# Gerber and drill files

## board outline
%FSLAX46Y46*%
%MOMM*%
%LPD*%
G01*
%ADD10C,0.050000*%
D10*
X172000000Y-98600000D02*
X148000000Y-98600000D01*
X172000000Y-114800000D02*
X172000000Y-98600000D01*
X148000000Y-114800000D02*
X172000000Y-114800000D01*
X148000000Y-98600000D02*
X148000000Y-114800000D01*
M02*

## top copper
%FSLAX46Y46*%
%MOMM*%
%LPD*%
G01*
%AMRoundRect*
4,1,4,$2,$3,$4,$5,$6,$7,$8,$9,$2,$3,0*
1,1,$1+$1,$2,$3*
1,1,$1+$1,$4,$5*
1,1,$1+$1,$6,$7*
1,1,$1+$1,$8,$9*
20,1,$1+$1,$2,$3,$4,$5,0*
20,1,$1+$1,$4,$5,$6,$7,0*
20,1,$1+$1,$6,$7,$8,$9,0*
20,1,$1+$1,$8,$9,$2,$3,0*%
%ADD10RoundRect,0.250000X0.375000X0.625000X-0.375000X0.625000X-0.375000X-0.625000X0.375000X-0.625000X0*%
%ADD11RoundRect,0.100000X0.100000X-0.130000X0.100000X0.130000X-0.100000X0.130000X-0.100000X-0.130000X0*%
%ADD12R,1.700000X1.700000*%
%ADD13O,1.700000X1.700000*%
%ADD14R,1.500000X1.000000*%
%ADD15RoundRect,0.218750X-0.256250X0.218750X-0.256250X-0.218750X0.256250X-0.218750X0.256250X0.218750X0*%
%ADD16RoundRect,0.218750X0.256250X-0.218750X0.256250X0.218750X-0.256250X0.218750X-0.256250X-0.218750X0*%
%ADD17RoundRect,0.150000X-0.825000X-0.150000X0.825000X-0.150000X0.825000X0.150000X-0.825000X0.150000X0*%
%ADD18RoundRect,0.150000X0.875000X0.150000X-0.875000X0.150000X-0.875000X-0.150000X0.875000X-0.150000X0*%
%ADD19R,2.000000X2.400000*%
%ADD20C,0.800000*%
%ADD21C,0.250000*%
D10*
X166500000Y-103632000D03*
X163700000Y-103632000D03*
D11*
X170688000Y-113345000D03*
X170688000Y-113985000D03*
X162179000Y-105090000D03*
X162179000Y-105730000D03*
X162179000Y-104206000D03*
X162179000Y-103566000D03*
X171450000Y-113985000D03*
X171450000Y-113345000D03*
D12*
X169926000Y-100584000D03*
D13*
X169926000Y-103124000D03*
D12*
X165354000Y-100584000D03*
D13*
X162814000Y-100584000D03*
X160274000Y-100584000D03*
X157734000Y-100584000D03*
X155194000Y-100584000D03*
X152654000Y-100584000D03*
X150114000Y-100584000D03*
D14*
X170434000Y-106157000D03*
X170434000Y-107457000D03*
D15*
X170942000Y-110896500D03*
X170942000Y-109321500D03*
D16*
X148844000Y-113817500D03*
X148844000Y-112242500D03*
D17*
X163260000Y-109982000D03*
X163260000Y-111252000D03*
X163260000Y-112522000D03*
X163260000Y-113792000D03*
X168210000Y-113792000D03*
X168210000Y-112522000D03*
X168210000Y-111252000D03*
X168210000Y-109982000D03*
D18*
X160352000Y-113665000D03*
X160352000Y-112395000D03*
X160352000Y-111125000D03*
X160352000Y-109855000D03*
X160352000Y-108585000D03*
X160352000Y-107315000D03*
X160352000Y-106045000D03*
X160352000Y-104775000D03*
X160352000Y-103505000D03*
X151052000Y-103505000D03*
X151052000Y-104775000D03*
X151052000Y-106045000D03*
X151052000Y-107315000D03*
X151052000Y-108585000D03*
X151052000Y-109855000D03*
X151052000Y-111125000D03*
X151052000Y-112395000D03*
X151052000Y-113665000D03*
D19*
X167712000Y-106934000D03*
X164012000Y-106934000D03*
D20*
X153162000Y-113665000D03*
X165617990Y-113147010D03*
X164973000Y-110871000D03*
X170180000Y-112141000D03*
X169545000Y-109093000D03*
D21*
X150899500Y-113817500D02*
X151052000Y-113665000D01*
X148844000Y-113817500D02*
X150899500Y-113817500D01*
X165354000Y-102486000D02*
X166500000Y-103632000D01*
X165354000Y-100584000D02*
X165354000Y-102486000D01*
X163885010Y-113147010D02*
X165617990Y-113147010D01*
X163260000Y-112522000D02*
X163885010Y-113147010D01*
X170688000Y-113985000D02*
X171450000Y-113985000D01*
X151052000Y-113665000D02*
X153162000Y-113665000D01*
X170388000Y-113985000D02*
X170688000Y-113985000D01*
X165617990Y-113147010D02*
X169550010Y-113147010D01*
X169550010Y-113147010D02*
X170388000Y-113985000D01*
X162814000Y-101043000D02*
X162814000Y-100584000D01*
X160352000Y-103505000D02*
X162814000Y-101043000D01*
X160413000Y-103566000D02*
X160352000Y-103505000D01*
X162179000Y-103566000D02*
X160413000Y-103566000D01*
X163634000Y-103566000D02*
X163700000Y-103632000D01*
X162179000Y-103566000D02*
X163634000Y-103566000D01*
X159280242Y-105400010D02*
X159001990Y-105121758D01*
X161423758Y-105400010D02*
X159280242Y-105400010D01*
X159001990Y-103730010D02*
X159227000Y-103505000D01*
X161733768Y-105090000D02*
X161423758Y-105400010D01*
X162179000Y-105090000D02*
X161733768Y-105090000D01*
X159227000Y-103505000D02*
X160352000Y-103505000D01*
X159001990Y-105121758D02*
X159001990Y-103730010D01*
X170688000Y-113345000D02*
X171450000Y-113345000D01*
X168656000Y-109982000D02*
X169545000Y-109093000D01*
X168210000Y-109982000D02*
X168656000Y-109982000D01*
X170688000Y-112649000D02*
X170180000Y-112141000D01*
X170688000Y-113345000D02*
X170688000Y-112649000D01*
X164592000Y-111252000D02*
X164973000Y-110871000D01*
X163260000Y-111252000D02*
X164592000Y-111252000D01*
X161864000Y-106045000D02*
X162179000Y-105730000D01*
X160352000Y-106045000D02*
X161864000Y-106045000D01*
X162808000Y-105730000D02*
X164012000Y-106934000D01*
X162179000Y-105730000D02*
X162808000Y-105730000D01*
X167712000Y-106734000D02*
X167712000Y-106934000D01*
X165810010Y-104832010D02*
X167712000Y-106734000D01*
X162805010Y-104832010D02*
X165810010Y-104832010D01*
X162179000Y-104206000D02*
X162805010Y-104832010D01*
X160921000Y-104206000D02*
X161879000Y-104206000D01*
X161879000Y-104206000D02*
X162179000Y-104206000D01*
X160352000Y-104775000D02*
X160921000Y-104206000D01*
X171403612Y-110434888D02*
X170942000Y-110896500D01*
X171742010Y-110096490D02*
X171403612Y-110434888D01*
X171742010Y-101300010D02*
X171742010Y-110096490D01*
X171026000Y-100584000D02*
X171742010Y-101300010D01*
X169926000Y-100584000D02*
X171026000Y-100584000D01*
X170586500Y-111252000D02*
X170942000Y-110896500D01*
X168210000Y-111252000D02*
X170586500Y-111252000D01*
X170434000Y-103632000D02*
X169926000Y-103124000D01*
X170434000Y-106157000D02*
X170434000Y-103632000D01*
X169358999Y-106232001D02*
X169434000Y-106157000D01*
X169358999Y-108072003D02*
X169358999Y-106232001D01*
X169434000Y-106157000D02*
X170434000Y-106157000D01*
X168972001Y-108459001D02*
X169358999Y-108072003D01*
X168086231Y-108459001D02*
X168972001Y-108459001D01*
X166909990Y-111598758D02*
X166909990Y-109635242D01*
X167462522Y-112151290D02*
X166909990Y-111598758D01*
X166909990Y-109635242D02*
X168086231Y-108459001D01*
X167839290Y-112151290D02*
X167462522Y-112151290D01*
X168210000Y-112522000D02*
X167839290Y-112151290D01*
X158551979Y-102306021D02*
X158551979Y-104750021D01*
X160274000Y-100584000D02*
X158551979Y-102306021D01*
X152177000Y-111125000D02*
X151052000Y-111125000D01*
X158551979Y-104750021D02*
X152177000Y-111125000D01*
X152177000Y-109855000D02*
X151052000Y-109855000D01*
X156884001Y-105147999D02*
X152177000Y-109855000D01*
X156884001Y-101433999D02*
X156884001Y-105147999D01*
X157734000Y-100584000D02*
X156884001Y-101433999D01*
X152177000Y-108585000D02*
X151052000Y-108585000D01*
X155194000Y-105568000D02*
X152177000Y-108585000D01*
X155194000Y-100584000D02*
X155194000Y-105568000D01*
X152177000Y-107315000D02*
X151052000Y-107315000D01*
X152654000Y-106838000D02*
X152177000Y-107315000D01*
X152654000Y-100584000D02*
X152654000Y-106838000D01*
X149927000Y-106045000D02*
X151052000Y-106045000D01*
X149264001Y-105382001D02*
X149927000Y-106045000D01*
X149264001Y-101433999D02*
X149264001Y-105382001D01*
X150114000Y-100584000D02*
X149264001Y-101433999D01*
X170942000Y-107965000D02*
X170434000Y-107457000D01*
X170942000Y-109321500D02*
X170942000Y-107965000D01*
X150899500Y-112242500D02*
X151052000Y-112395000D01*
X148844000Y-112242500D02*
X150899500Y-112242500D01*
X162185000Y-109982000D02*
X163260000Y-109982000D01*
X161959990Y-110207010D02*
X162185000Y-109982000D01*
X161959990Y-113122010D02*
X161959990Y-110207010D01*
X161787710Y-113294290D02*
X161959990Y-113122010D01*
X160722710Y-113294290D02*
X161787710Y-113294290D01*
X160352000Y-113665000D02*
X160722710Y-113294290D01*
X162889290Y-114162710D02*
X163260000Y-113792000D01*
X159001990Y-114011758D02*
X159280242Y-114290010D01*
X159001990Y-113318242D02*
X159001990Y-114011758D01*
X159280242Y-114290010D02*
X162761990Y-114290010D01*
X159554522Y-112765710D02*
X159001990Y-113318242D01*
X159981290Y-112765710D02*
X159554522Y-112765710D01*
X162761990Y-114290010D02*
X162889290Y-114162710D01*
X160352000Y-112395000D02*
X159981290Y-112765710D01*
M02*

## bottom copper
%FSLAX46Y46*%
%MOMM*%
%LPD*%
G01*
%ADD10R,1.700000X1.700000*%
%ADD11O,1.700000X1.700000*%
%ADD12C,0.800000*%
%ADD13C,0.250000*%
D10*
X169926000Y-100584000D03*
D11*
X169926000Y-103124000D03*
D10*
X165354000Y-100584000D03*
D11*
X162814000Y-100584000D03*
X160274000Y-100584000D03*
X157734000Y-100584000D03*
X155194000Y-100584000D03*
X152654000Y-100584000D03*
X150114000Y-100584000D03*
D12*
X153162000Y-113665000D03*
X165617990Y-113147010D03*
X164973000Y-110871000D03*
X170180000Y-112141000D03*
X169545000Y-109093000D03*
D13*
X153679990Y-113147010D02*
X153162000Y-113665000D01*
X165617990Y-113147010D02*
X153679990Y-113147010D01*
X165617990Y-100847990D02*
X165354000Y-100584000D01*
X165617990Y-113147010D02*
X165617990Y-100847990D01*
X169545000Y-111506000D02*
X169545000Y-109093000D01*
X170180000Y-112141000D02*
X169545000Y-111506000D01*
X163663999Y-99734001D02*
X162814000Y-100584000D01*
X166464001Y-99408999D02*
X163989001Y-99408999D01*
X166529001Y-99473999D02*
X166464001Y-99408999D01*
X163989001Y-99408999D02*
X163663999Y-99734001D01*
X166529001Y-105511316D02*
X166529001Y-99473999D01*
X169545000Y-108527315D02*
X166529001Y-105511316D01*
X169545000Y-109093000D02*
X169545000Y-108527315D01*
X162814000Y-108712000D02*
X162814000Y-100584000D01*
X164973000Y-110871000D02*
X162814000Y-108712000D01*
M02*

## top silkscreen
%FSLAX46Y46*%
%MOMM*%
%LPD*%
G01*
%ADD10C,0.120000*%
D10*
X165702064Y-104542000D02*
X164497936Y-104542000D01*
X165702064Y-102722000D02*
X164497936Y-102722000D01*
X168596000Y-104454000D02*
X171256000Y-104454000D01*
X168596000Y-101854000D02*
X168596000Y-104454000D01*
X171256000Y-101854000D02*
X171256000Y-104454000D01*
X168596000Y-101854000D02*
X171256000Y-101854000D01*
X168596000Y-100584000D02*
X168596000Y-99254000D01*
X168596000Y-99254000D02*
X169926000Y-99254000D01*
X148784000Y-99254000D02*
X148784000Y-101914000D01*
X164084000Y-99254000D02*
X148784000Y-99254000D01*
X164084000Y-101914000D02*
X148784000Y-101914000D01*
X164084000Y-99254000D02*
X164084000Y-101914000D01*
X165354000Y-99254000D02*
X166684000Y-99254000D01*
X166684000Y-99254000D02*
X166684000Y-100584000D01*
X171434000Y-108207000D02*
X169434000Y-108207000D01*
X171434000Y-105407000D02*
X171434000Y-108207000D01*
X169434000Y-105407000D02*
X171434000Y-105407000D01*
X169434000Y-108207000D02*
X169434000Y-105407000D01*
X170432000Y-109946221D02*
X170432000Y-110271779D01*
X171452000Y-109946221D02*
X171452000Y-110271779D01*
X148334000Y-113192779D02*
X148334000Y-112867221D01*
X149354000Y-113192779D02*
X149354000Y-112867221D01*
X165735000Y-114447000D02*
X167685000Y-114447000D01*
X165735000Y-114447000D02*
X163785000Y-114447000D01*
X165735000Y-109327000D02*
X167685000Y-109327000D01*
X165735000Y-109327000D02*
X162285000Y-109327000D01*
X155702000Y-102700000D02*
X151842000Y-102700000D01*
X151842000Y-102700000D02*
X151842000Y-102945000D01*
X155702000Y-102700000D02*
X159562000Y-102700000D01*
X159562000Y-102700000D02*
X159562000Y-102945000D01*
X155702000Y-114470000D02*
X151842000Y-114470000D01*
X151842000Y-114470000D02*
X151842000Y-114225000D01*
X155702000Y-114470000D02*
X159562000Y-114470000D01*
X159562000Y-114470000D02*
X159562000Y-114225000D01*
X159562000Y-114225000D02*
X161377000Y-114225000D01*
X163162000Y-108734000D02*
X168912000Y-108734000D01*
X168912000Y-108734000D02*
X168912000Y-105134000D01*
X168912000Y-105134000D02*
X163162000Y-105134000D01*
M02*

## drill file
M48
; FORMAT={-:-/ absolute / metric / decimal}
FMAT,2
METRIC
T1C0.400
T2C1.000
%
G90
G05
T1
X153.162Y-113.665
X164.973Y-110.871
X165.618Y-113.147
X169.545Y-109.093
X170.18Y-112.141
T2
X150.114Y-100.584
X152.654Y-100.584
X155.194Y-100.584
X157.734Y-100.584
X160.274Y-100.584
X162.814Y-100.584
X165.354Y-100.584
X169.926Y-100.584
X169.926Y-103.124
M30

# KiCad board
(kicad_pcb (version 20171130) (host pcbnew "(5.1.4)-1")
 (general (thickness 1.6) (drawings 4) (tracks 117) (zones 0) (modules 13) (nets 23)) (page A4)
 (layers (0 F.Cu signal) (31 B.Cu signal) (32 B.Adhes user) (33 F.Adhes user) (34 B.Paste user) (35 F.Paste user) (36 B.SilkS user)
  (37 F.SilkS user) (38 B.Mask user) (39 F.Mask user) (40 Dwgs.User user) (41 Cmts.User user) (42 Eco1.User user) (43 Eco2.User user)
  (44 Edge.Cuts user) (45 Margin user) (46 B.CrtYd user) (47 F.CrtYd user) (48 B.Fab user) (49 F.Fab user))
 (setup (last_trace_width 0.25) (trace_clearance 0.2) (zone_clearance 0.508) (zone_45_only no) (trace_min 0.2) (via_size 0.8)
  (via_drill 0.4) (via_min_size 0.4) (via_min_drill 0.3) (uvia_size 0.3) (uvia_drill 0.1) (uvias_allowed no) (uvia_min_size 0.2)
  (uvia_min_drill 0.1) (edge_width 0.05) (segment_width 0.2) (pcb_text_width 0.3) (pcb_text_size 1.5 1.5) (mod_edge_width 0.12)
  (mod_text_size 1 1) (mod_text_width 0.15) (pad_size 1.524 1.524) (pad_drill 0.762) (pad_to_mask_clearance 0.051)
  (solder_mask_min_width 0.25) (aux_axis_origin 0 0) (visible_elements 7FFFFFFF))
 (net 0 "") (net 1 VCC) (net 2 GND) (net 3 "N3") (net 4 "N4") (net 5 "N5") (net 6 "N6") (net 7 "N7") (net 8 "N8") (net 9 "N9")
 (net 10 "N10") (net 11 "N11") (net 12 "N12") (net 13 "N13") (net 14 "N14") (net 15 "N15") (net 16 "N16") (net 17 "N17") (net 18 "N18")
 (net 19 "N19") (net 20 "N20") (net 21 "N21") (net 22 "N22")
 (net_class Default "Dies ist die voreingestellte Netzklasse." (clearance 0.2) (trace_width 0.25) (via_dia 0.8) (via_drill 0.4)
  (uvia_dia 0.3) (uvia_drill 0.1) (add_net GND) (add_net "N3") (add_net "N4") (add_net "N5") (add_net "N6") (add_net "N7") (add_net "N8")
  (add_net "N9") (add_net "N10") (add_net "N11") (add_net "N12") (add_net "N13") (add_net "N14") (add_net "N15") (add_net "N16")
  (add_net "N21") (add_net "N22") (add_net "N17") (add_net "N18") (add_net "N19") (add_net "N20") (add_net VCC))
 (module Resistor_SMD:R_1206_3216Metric (layer F.Cu) (at 165.1 103.632 180)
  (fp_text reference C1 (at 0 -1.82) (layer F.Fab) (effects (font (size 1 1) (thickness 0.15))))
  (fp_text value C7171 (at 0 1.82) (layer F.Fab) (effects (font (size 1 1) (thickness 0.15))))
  (fp_line (start -0.602064 -0.91) (end 0.602064 -0.91) (layer F.SilkS) (width 0.12))
  (fp_line (start -0.602064 0.91) (end 0.602064 0.91) (layer F.SilkS) (width 0.12))
  (pad 1 smd roundrect (at -1.4 0 180) (size 1.25 1.75) (layers F.Cu F.Paste F.Mask) (roundrect_rratio 0.2) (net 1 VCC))
  (pad 2 smd roundrect (at 1.4 0 180) (size 1.25 1.75) (layers F.Cu F.Paste F.Mask) (roundrect_rratio 0.2) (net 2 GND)))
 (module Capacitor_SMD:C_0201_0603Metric (layer F.Cu) (at 170.688 113.665 90)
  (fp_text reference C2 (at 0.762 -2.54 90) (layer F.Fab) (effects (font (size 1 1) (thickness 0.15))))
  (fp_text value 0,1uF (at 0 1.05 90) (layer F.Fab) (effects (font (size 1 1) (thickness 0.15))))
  (pad 2 smd roundrect (at 0.32 0 90) (size 0.46 0.4) (layers F.Cu F.Mask) (roundrect_rratio 0.25) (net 2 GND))
  (pad 1 smd roundrect (at -0.32 0 90) (size 0.46 0.4) (layers F.Cu F.Mask) (roundrect_rratio 0.25) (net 1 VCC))
  (pad "" smd roundrect (at 0.345 0 90) (size 0.318 0.36) (layers F.Paste) (roundrect_rratio 0.25))
  (pad "" smd roundrect (at -0.345 0 90) (size 0.318 0.36) (layers F.Paste) (roundrect_rratio 0.25)))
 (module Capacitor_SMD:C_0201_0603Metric (layer F.Cu) (at 162.179 105.41 90)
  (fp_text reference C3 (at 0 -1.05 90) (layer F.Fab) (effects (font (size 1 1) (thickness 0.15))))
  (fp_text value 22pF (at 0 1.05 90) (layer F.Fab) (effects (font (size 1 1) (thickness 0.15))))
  (pad 2 smd roundrect (at 0.32 0 90) (size 0.46 0.4) (layers F.Cu F.Mask) (roundrect_rratio 0.25) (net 2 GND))
  (pad 1 smd roundrect (at -0.32 0 90) (size 0.46 0.4) (layers F.Cu F.Mask) (roundrect_rratio 0.25) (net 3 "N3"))
  (pad "" smd roundrect (at 0.345 0 90) (size 0.318 0.36) (layers F.Paste) (roundrect_rratio 0.25))
  (pad "" smd roundrect (at -0.345 0 90) (size 0.318 0.36) (layers F.Paste) (roundrect_rratio 0.25)))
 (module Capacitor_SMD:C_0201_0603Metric (layer F.Cu) (at 162.179 103.886 90)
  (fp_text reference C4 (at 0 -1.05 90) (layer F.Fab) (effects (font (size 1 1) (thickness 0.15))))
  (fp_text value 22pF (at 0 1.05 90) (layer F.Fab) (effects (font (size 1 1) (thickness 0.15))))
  (pad "" smd roundrect (at -0.345 0 90) (size 0.318 0.36) (layers F.Paste) (roundrect_rratio 0.25))
  (pad "" smd roundrect (at 0.345 0 90) (size 0.318 0.36) (layers F.Paste) (roundrect_rratio 0.25))
  (pad 1 smd roundrect (at -0.32 0 90) (size 0.46 0.4) (layers F.Cu F.Mask) (roundrect_rratio 0.25) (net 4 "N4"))
  (pad 2 smd roundrect (at 0.32 0 90) (size 0.46 0.4) (layers F.Cu F.Mask) (roundrect_rratio 0.25) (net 2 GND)))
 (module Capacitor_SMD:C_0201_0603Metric (layer F.Cu) (at 171.45 113.665 90)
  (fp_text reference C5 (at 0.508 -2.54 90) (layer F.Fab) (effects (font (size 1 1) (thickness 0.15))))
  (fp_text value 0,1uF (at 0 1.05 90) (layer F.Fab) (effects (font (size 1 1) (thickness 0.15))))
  (pad "" smd roundrect (at -0.345 0 90) (size 0.318 0.36) (layers F.Paste) (roundrect_rratio 0.25))
  (pad "" smd roundrect (at 0.345 0 90) (size 0.318 0.36) (layers F.Paste) (roundrect_rratio 0.25))
  (pad 1 smd roundrect (at -0.32 0 90) (size 0.46 0.4) (layers F.Cu F.Mask) (roundrect_rratio 0.25) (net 1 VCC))
  (pad 2 smd roundrect (at 0.32 0 90) (size 0.46 0.4) (layers F.Cu F.Mask) (roundrect_rratio 0.25) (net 2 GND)))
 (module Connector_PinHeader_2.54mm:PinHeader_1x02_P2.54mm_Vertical (layer F.Cu) (at 169.926 100.584)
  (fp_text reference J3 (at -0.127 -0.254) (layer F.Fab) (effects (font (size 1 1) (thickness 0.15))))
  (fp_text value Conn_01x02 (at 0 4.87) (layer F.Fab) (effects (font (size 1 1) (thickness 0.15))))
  (fp_line (start -1.33 3.87) (end 1.33 3.87) (layer F.SilkS) (width 0.12))
  (fp_line (start -1.33 1.27) (end -1.33 3.87) (layer F.SilkS) (width 0.12))
  (fp_line (start 1.33 1.27) (end 1.33 3.87) (layer F.SilkS) (width 0.12))
  (fp_line (start -1.33 1.27) (end 1.33 1.27) (layer F.SilkS) (width 0.12))
  (fp_line (start -1.33 0) (end -1.33 -1.33) (layer F.SilkS) (width 0.12))
  (fp_line (start -1.33 -1.33) (end 0 -1.33) (layer F.SilkS) (width 0.12))
  (pad 1 thru_hole rect (at 0 0) (size 1.7 1.7) (drill 1) (layers *.Cu *.Mask) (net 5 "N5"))
  (pad 2 thru_hole oval (at 0 2.54) (size 1.7 1.7) (drill 1) (layers *.Cu *.Mask) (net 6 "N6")))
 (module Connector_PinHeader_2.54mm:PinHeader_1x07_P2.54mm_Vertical (layer F.Cu) (at 165.354 100.584 270)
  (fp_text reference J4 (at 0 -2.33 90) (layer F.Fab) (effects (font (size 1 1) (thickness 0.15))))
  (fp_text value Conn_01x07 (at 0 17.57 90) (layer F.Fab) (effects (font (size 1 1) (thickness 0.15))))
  (fp_line (start -1.33 16.57) (end 1.33 16.57) (layer F.SilkS) (width 0.12))
  (fp_line (start -1.33 1.27) (end -1.33 16.57) (layer F.SilkS) (width 0.12))
  (fp_line (start 1.33 1.27) (end 1.33 16.57) (layer F.SilkS) (width 0.12))
  (fp_line (start -1.33 1.27) (end 1.33 1.27) (layer F.SilkS) (width 0.12))
  (fp_line (start -1.33 0) (end -1.33 -1.33) (layer F.SilkS) (width 0.12))
  (fp_line (start -1.33 -1.33) (end 0 -1.33) (layer F.SilkS) (width 0.12))
  (pad 1 thru_hole rect (at 0 0 270) (size 1.7 1.7) (drill 1) (layers *.Cu *.Mask) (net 1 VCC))
  (pad 2 thru_hole oval (at 0 2.54 270) (size 1.7 1.7) (drill 1) (layers *.Cu *.Mask) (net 2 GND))
  (pad 3 thru_hole oval (at 0 5.08 270) (size 1.7 1.7) (drill 1) (layers *.Cu *.Mask) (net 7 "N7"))
  (pad 4 thru_hole oval (at 0 7.62 270) (size 1.7 1.7) (drill 1) (layers *.Cu *.Mask) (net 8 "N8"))
  (pad 5 thru_hole oval (at 0 10.16 270) (size 1.7 1.7) (drill 1) (layers *.Cu *.Mask) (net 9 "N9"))
  (pad 6 thru_hole oval (at 0 12.7 270) (size 1.7 1.7) (drill 1) (layers *.Cu *.Mask) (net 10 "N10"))
  (pad 7 thru_hole oval (at 0 15.24 270) (size 1.7 1.7) (drill 1) (layers *.Cu *.Mask) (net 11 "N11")))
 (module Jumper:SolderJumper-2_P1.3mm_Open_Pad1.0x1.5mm (layer F.Cu) (at 170.434 106.807 90)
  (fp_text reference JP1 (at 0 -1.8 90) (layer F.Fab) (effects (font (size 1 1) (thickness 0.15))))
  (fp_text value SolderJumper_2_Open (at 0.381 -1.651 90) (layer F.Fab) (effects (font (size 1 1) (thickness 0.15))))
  (fp_line (start -1.4 1) (end -1.4 -1) (layer F.SilkS) (width 0.12))
  (fp_line (start 1.4 1) (end -1.4 1) (layer F.SilkS) (width 0.12))
  (fp_line (start 1.4 -1) (end 1.4 1) (layer F.SilkS) (width 0.12))
  (fp_line (start -1.4 -1) (end 1.4 -1) (layer F.SilkS) (width 0.12))
  (pad 2 smd rect (at 0.65 0 90) (size 1 1.5) (layers F.Cu F.Mask) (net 6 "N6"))
  (pad 1 smd rect (at -0.65 0 90) (size 1 1.5) (layers F.Cu F.Mask) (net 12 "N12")))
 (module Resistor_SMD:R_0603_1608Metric (layer F.Cu) (at 170.942 110.109 270)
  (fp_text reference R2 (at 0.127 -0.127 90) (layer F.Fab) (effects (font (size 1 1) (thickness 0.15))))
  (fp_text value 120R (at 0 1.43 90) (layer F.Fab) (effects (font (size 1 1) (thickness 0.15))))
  (fp_line (start -0.162779 0.51) (end 0.162779 0.51) (layer F.SilkS) (width 0.12))
  (fp_line (start -0.162779 -0.51) (end 0.162779 -0.51) (layer F.SilkS) (width 0.12))
  (pad 2 smd roundrect (at 0.7875 0 270) (size 0.875 0.95) (layers F.Cu F.Paste F.Mask) (roundrect_rratio 0.25) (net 5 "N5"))
  (pad 1 smd roundrect (at -0.7875 0 270) (size 0.875 0.95) (layers F.Cu F.Paste F.Mask) (roundrect_rratio 0.25) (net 12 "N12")))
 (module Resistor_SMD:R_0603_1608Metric (layer F.Cu) (at 148.844 113.03 90)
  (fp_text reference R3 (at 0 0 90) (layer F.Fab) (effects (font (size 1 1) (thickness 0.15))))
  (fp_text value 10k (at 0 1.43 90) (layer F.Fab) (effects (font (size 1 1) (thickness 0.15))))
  (fp_line (start -0.162779 -0.51) (end 0.162779 -0.51) (layer F.SilkS) (width 0.12))
  (fp_line (start -0.162779 0.51) (end 0.162779 0.51) (layer F.SilkS) (width 0.12))
  (pad 1 smd roundrect (at -0.7875 0 90) (size 0.875 0.95) (layers F.Cu F.Paste F.Mask) (roundrect_rratio 0.25) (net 1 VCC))
  (pad 2 smd roundrect (at 0.7875 0 90) (size 0.875 0.95) (layers F.Cu F.Paste F.Mask) (roundrect_rratio 0.25) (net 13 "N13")))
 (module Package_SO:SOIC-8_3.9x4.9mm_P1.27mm (layer F.Cu) (at 165.735 111.887)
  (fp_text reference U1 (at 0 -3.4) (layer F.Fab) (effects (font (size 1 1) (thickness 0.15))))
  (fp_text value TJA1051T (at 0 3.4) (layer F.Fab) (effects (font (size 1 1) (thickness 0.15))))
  (fp_line (start 0 2.56) (end 1.95 2.56) (layer F.SilkS) (width 0.12))
  (fp_line (start 0 2.56) (end -1.95 2.56) (layer F.SilkS) (width 0.12))
  (fp_line (start 0 -2.56) (end 1.95 -2.56) (layer F.SilkS) (width 0.12))
  (fp_line (start 0 -2.56) (end -3.45 -2.56) (layer F.SilkS) (width 0.12))
  (pad 1 smd roundrect (at -2.475 -1.905) (size 1.95 0.6) (layers F.Cu F.Paste F.Mask) (roundrect_rratio 0.25) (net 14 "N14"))
  (pad 2 smd roundrect (at -2.475 -0.635) (size 1.95 0.6) (layers F.Cu F.Paste F.Mask) (roundrect_rratio 0.25) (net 2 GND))
  (pad 3 smd roundrect (at -2.475 0.635) (size 1.95 0.6) (layers F.Cu F.Paste F.Mask) (roundrect_rratio 0.25) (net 1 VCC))
  (pad 4 smd roundrect (at -2.475 1.905) (size 1.95 0.6) (layers F.Cu F.Paste F.Mask) (roundrect_rratio 0.25) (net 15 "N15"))
  (pad 5 smd roundrect (at 2.475 1.905) (size 1.95 0.6) (layers F.Cu F.Paste F.Mask) (roundrect_rratio 0.25) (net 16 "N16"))
  (pad 6 smd roundrect (at 2.475 0.635) (size 1.95 0.6) (layers F.Cu F.Paste F.Mask) (roundrect_rratio 0.25) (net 6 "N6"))
  (pad 7 smd roundrect (at 2.475 -0.635) (size 1.95 0.6) (layers F.Cu F.Paste F.Mask) (roundrect_rratio 0.25) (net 5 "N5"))
  (pad 8 smd roundrect (at 2.475 -1.905) (size 1.95 0.6) (layers F.Cu F.Paste F.Mask) (roundrect_rratio 0.25) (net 2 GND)))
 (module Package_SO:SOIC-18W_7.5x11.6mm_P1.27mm (layer F.Cu) (at 155.702 108.585 180)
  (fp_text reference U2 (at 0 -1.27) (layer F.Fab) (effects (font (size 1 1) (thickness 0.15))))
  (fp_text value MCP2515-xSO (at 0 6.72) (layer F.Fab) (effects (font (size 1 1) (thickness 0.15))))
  (fp_line (start 0 5.885) (end 3.86 5.885) (layer F.SilkS) (width 0.12))
  (fp_line (start 3.86 5.885) (end 3.86 5.64) (layer F.SilkS) (width 0.12))
  (fp_line (start 0 5.885) (end -3.86 5.885) (layer F.SilkS) (width 0.12))
  (fp_line (start -3.86 5.885) (end -3.86 5.64) (layer F.SilkS) (width 0.12))
  (fp_line (start 0 -5.885) (end 3.86 -5.885) (layer F.SilkS) (width 0.12))
  (fp_line (start 3.86 -5.885) (end 3.86 -5.64) (layer F.SilkS) (width 0.12))
  (fp_line (start 0 -5.885) (end -3.86 -5.885) (layer F.SilkS) (width 0.12))
  (fp_line (start -3.86 -5.885) (end -3.86 -5.64) (layer F.SilkS) (width 0.12))
  (fp_line (start -3.86 -5.64) (end -5.675 -5.64) (layer F.SilkS) (width 0.12))
  (pad 1 smd roundrect (at -4.65 -5.08 180) (size 2.05 0.6) (layers F.Cu F.Paste F.Mask) (roundrect_rratio 0.25) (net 14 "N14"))
  (pad 2 smd roundrect (at -4.65 -3.81 180) (size 2.05 0.6) (layers F.Cu F.Paste F.Mask) (roundrect_rratio 0.25) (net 15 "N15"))
  (pad 3 smd roundrect (at -4.65 -2.54 180) (size 2.05 0.6) (layers F.Cu F.Paste F.Mask) (roundrect_rratio 0.25) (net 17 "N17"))
  (pad 4 smd roundrect (at -4.65 -1.27 180) (size 2.05 0.6) (layers F.Cu F.Paste F.Mask) (roundrect_rratio 0.25) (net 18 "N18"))
  (pad 5 smd roundrect (at -4.65 0 180) (size 2.05 0.6) (layers F.Cu F.Paste F.Mask) (roundrect_rratio 0.25) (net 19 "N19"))
  (pad 6 smd roundrect (at -4.65 1.27 180) (size 2.05 0.6) (layers F.Cu F.Paste F.Mask) (roundrect_rratio 0.25) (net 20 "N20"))
  (pad 7 smd roundrect (at -4.65 2.54 180) (size 2.05 0.6) (layers F.Cu F.Paste F.Mask) (roundrect_rratio 0.25) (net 3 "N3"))
  (pad 8 smd roundrect (at -4.65 3.81 180) (size 2.05 0.6) (layers F.Cu F.Paste F.Mask) (roundrect_rratio 0.25) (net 4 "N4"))
  (pad 9 smd roundrect (at -4.65 5.08 180) (size 2.05 0.6) (layers F.Cu F.Paste F.Mask) (roundrect_rratio 0.25) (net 2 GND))
  (pad 10 smd roundrect (at 4.65 5.08 180) (size 2.05 0.6) (layers F.Cu F.Paste F.Mask) (roundrect_rratio 0.25) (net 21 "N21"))
  (pad 11 smd roundrect (at 4.65 3.81 180) (size 2.05 0.6) (layers F.Cu F.Paste F.Mask) (roundrect_rratio 0.25) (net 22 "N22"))
  (pad 12 smd roundrect (at 4.65 2.54 180) (size 2.05 0.6) (layers F.Cu F.Paste F.Mask) (roundrect_rratio 0.25) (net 11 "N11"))
  (pad 13 smd roundrect (at 4.65 1.27 180) (size 2.05 0.6) (layers F.Cu F.Paste F.Mask) (roundrect_rratio 0.25) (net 10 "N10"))
  (pad 14 smd roundrect (at 4.65 0 180) (size 2.05 0.6) (layers F.Cu F.Paste F.Mask) (roundrect_rratio 0.25) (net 9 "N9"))
  (pad 15 smd roundrect (at 4.65 -1.27 180) (size 2.05 0.6) (layers F.Cu F.Paste F.Mask) (roundrect_rratio 0.25) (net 8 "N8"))
  (pad 16 smd roundrect (at 4.65 -2.54 180) (size 2.05 0.6) (layers F.Cu F.Paste F.Mask) (roundrect_rratio 0.25) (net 7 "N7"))
  (pad 17 smd roundrect (at 4.65 -3.81 180) (size 2.05 0.6) (layers F.Cu F.Paste F.Mask) (roundrect_rratio 0.25) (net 13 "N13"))
  (pad 18 smd roundrect (at 4.65 -5.08 180) (size 2.05 0.6) (layers F.Cu F.Paste F.Mask) (roundrect_rratio 0.25) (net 1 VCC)))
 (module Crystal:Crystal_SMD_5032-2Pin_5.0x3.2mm (layer F.Cu) (at 165.862 106.934 180)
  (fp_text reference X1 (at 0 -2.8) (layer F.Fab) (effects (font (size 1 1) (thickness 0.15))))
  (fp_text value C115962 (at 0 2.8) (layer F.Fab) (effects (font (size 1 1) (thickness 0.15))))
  (fp_line (start 2.7 -1.8) (end -3.05 -1.8) (layer F.SilkS) (width 0.12))
  (fp_line (start -3.05 -1.8) (end -3.05 1.8) (layer F.SilkS) (width 0.12))
  (fp_line (start -3.05 1.8) (end 2.7 1.8) (layer F.SilkS) (width 0.12))
  (pad 1 smd rect (at -1.85 0 180) (size 2 2.4) (layers F.Cu F.Paste F.Mask) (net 4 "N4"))
  (pad 2 smd rect (at 1.85 0 180) (size 2 2.4) (layers F.Cu F.Paste F.Mask) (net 3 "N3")))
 (gr_line (start 172 98.6) (end 148 98.6) (layer Edge.Cuts) (width 0.05))
 (gr_line (start 172 114.8) (end 172 98.6) (layer Edge.Cuts) (width 0.05))
 (gr_line (start 148 114.8) (end 172 114.8) (layer Edge.Cuts) (width 0.05))
 (gr_line (start 148 98.6) (end 148 114.8) (layer Edge.Cuts) (width 0.05))
 (via (at 153.162 113.665) (size 0.8) (drill 0.4) (layers F.Cu B.Cu) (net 1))
 (segment (start 150.8995 113.8175) (end 151.052 113.665) (width 0.25) (layer F.Cu) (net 1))
 (segment (start 148.844 113.8175) (end 150.8995 113.8175) (width 0.25) (layer F.Cu) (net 1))
 (segment (start 165.354 102.486) (end 166.5 103.632) (width 0.25) (layer F.Cu) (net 1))
 (segment (start 165.354 100.584) (end 165.354 102.486) (width 0.25) (layer F.Cu) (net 1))
 (segment (start 163.88501 113.14701) (end 165.61799 113.14701) (width 0.25) (layer F.Cu) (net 1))
 (segment (start 163.26 112.522) (end 163.88501 113.14701) (width 0.25) (layer F.Cu) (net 1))
 (segment (start 170.688 113.985) (end 171.45 113.985) (width 0.25) (layer F.Cu) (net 1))
 (via (at 165.61799 113.14701) (size 0.8) (drill 0.4) (layers F.Cu B.Cu) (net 1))
 (segment (start 151.052 113.665) (end 153.162 113.665) (width 0.25) (layer F.Cu) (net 1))
 (segment (start 153.67999 113.14701) (end 153.162 113.665) (width 0.25) (layer B.Cu) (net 1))
 (segment (start 165.61799 113.14701) (end 153.67999 113.14701) (width 0.25) (layer B.Cu) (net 1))
 (segment (start 165.61799 100.84799) (end 165.354 100.584) (width 0.25) (layer B.Cu) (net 1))
 (segment (start 165.61799 113.14701) (end 165.61799 100.84799) (width 0.25) (layer B.Cu) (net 1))
 (segment (start 170.388 113.985) (end 170.688 113.985) (width 0.25) (layer F.Cu) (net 1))
 (segment (start 165.61799 113.14701) (end 169.55001 113.14701) (width 0.25) (layer F.Cu) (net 1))
 (segment (start 169.55001 113.14701) (end 170.388 113.985) (width 0.25) (layer F.Cu) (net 1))
 (via (at 164.973 110.871) (size 0.8) (drill 0.4) (layers F.Cu B.Cu) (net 2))
 (via (at 170.18 112.141) (size 0.8) (drill 0.4) (layers F.Cu B.Cu) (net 2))
 (via (at 169.545 109.093) (size 0.8) (drill 0.4) (layers F.Cu B.Cu) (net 2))
 (segment (start 162.814 101.043) (end 162.814 100.584) (width 0.25) (layer F.Cu) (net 2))
 (segment (start 160.352 103.505) (end 162.814 101.043) (width 0.25) (layer F.Cu) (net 2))
 (segment (start 160.413 103.566) (end 160.352 103.505) (width 0.25) (layer F.Cu) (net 2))
 (segment (start 162.179 103.566) (end 160.413 103.566) (width 0.25) (layer F.Cu) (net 2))
 (segment (start 163.634 103.566) (end 163.7 103.632) (width 0.25) (layer F.Cu) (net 2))
 (segment (start 162.179 103.566) (end 163.634 103.566) (width 0.25) (layer F.Cu) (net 2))
 (segment (start 159.280242 105.40001) (end 159.00199 105.121758) (width 0.25) (layer F.Cu) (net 2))
 (segment (start 161.423758 105.40001) (end 159.280242 105.40001) (width 0.25) (layer F.Cu) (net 2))
 (segment (start 159.00199 103.73001) (end 159.227 103.505) (width 0.25) (layer F.Cu) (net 2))
 (segment (start 161.733768 105.09) (end 161.423758 105.40001) (width 0.25) (layer F.Cu) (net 2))
 (segment (start 162.179 105.09) (end 161.733768 105.09) (width 0.25) (layer F.Cu) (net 2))
 (segment (start 159.227 103.505) (end 160.352 103.505) (width 0.25) (layer F.Cu) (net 2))
 (segment (start 159.00199 105.121758) (end 159.00199 103.73001) (width 0.25) (layer F.Cu) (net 2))
 (segment (start 170.688 113.345) (end 171.45 113.345) (width 0.25) (layer F.Cu) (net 2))
 (segment (start 168.656 109.982) (end 169.545 109.093) (width 0.25) (layer F.Cu) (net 2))
 (segment (start 168.21 109.982) (end 168.656 109.982) (width 0.25) (layer F.Cu) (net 2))
 (segment (start 170.688 112.649) (end 170.18 112.141) (width 0.25) (layer F.Cu) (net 2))
 (segment (start 170.688 113.345) (end 170.688 112.649) (width 0.25) (layer F.Cu) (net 2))
 (segment (start 169.545 111.506) (end 169.545 109.093) (width 0.25) (layer B.Cu) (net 2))
 (segment (start 170.18 112.141) (end 169.545 111.506) (width 0.25) (layer B.Cu) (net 2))
 (segment (start 163.663999 99.734001) (end 162.814 100.584) (width 0.25) (layer B.Cu) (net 2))
 (segment (start 166.464001 99.408999) (end 163.989001 99.408999) (width 0.25) (layer B.Cu) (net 2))
 (segment (start 166.529001 99.473999) (end 166.464001 99.408999) (width 0.25) (layer B.Cu) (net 2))
 (segment (start 163.989001 99.408999) (end 163.663999 99.734001) (width 0.25) (layer B.Cu) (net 2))
 (segment (start 166.529001 105.511316) (end 166.529001 99.473999) (width 0.25) (layer B.Cu) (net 2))
 (segment (start 169.545 108.527315) (end 166.529001 105.511316) (width 0.25) (layer B.Cu) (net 2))
 (segment (start 169.545 109.093) (end 169.545 108.527315) (width 0.25) (layer B.Cu) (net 2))
 (segment (start 162.814 108.712) (end 162.814 100.584) (width 0.25) (layer B.Cu) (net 2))
 (segment (start 164.973 110.871) (end 162.814 108.712) (width 0.25) (layer B.Cu) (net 2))
 (segment (start 164.592 111.252) (end 164.973 110.871) (width 0.25) (layer F.Cu) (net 2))
 (segment (start 163.26 111.252) (end 164.592 111.252) (width 0.25) (layer F.Cu) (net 2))
 (segment (start 161.864 106.045) (end 162.179 105.73) (width 0.25) (layer F.Cu) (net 3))
 (segment (start 160.352 106.045) (end 161.864 106.045) (width 0.25) (layer F.Cu) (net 3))
 (segment (start 162.808 105.73) (end 164.012 106.934) (width 0.25) (layer F.Cu) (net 3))
 (segment (start 162.179 105.73) (end 162.808 105.73) (width 0.25) (layer F.Cu) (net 3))
 (segment (start 167.712 106.734) (end 167.712 106.934) (width 0.25) (layer F.Cu) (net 4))
 (segment (start 165.81001 104.83201) (end 167.712 106.734) (width 0.25) (layer F.Cu) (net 4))
 (segment (start 162.80501 104.83201) (end 165.81001 104.83201) (width 0.25) (layer F.Cu) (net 4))
 (segment (start 162.179 104.206) (end 162.80501 104.83201) (width 0.25) (layer F.Cu) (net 4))
 (segment (start 160.921 104.206) (end 161.879 104.206) (width 0.25) (layer F.Cu) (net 4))
 (segment (start 161.879 104.206) (end 162.179 104.206) (width 0.25) (layer F.Cu) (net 4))
 (segment (start 160.352 104.775) (end 160.921 104.206) (width 0.25) (layer F.Cu) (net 4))
 (segment (start 171.403612 110.434888) (end 170.942 110.8965) (width 0.25) (layer F.Cu) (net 5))
 (segment (start 171.74201 110.09649) (end 171.403612 110.434888) (width 0.25) (layer F.Cu) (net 5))
 (segment (start 171.74201 101.30001) (end 171.74201 110.09649) (width 0.25) (layer F.Cu) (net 5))
 (segment (start 171.026 100.584) (end 171.74201 101.30001) (width 0.25) (layer F.Cu) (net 5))
 (segment (start 169.926 100.584) (end 171.026 100.584) (width 0.25) (layer F.Cu) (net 5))
 (segment (start 170.5865 111.252) (end 170.942 110.8965) (width 0.25) (layer F.Cu) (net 5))
 (segment (start 168.21 111.252) (end 170.5865 111.252) (width 0.25) (layer F.Cu) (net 5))
 (segment (start 170.434 103.632) (end 169.926 103.124) (width 0.25) (layer F.Cu) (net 6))
 (segment (start 170.434 106.157) (end 170.434 103.632) (width 0.25) (layer F.Cu) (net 6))
 (segment (start 169.358999 106.232001) (end 169.434 106.157) (width 0.25) (layer F.Cu) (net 6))
 (segment (start 169.358999 108.072003) (end 169.358999 106.232001) (width 0.25) (layer F.Cu) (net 6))
 (segment (start 169.434 106.157) (end 170.434 106.157) (width 0.25) (layer F.Cu) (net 6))
 (segment (start 168.972001 108.459001) (end 169.358999 108.072003) (width 0.25) (layer F.Cu) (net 6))
 (segment (start 168.086231 108.459001) (end 168.972001 108.459001) (width 0.25) (layer F.Cu) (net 6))
 (segment (start 166.90999 111.598758) (end 166.90999 109.635242) (width 0.25) (layer F.Cu) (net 6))
 (segment (start 167.462522 112.15129) (end 166.90999 111.598758) (width 0.25) (layer F.Cu) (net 6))
 (segment (start 166.90999 109.635242) (end 168.086231 108.459001) (width 0.25) (layer F.Cu) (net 6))
 (segment (start 167.83929 112.15129) (end 167.462522 112.15129) (width 0.25) (layer F.Cu) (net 6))
 (segment (start 168.21 112.522) (end 167.83929 112.15129) (width 0.25) (layer F.Cu) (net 6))
 (segment (start 158.551979 102.306021) (end 158.551979 104.750021) (width 0.25) (layer F.Cu) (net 7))
 (segment (start 160.274 100.584) (end 158.551979 102.306021) (width 0.25) (layer F.Cu) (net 7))
 (segment (start 152.177 111.125) (end 151.052 111.125) (width 0.25) (layer F.Cu) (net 7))
 (segment (start 158.551979 104.750021) (end 152.177 111.125) (width 0.25) (layer F.Cu) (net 7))
 (segment (start 152.177 109.855) (end 151.052 109.855) (width 0.25) (layer F.Cu) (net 8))
 (segment (start 156.884001 105.147999) (end 152.177 109.855) (width 0.25) (layer F.Cu) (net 8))
 (segment (start 156.884001 101.433999) (end 156.884001 105.147999) (width 0.25) (layer F.Cu) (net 8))
 (segment (start 157.734 100.584) (end 156.884001 101.433999) (width 0.25) (layer F.Cu) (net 8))
 (segment (start 152.177 108.585) (end 151.052 108.585) (width 0.25) (layer F.Cu) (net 9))
 (segment (start 155.194 105.568) (end 152.177 108.585) (width 0.25) (layer F.Cu) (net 9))
 (segment (start 155.194 100.584) (end 155.194 105.568) (width 0.25) (layer F.Cu) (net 9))
 (segment (start 152.177 107.315) (end 151.052 107.315) (width 0.25) (layer F.Cu) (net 10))
 (segment (start 152.654 106.838) (end 152.177 107.315) (width 0.25) (layer F.Cu) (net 10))
 (segment (start 152.654 100.584) (end 152.654 106.838) (width 0.25) (layer F.Cu) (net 10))
 (segment (start 149.927 106.045) (end 151.052 106.045) (width 0.25) (layer F.Cu) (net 11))
 (segment (start 149.264001 105.382001) (end 149.927 106.045) (width 0.25) (layer F.Cu) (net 11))
 (segment (start 149.264001 101.433999) (end 149.264001 105.382001) (width 0.25) (layer F.Cu) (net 11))
 (segment (start 150.114 100.584) (end 149.264001 101.433999) (width 0.25) (layer F.Cu) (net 11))
 (segment (start 170.942 107.965) (end 170.434 107.457) (width 0.25) (layer F.Cu) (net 12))
 (segment (start 170.942 109.3215) (end 170.942 107.965) (width 0.25) (layer F.Cu) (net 12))
 (segment (start 150.8995 112.2425) (end 151.052 112.395) (width 0.25) (layer F.Cu) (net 13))
 (segment (start 148.844 112.2425) (end 150.8995 112.2425) (width 0.25) (layer F.Cu) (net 13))
 (segment (start 162.185 109.982) (end 163.26 109.982) (width 0.25) (layer F.Cu) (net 14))
 (segment (start 161.95999 110.20701) (end 162.185 109.982) (width 0.25) (layer F.Cu) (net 14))
 (segment (start 161.95999 113.12201) (end 161.95999 110.20701) (width 0.25) (layer F.Cu) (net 14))
 (segment (start 161.78771 113.29429) (end 161.95999 113.12201) (width 0.25) (layer F.Cu) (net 14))
 (segment (start 160.72271 113.29429) (end 161.78771 113.29429) (width 0.25) (layer F.Cu) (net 14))
 (segment (start 160.352 113.665) (end 160.72271 113.29429) (width 0.25) (layer F.Cu) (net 14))
 (segment (start 162.88929 114.16271) (end 163.26 113.792) (width 0.25) (layer F.Cu) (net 15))
 (segment (start 159.00199 114.011758) (end 159.280242 114.29001) (width 0.25) (layer F.Cu) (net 15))
 (segment (start 159.00199 113.318242) (end 159.00199 114.011758) (width 0.25) (layer F.Cu) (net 15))
 (segment (start 159.280242 114.29001) (end 162.76199 114.29001) (width 0.25) (layer F.Cu) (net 15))
 (segment (start 159.554522 112.76571) (end 159.00199 113.318242) (width 0.25) (layer F.Cu) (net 15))
 (segment (start 159.98129 112.76571) (end 159.554522 112.76571) (width 0.25) (layer F.Cu) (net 15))
 (segment (start 162.76199 114.29001) (end 162.88929 114.16271) (width 0.25) (layer F.Cu) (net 15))
 (segment (start 160.352 112.395) (end 159.98129 112.76571) (width 0.25) (layer F.Cu) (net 15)))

